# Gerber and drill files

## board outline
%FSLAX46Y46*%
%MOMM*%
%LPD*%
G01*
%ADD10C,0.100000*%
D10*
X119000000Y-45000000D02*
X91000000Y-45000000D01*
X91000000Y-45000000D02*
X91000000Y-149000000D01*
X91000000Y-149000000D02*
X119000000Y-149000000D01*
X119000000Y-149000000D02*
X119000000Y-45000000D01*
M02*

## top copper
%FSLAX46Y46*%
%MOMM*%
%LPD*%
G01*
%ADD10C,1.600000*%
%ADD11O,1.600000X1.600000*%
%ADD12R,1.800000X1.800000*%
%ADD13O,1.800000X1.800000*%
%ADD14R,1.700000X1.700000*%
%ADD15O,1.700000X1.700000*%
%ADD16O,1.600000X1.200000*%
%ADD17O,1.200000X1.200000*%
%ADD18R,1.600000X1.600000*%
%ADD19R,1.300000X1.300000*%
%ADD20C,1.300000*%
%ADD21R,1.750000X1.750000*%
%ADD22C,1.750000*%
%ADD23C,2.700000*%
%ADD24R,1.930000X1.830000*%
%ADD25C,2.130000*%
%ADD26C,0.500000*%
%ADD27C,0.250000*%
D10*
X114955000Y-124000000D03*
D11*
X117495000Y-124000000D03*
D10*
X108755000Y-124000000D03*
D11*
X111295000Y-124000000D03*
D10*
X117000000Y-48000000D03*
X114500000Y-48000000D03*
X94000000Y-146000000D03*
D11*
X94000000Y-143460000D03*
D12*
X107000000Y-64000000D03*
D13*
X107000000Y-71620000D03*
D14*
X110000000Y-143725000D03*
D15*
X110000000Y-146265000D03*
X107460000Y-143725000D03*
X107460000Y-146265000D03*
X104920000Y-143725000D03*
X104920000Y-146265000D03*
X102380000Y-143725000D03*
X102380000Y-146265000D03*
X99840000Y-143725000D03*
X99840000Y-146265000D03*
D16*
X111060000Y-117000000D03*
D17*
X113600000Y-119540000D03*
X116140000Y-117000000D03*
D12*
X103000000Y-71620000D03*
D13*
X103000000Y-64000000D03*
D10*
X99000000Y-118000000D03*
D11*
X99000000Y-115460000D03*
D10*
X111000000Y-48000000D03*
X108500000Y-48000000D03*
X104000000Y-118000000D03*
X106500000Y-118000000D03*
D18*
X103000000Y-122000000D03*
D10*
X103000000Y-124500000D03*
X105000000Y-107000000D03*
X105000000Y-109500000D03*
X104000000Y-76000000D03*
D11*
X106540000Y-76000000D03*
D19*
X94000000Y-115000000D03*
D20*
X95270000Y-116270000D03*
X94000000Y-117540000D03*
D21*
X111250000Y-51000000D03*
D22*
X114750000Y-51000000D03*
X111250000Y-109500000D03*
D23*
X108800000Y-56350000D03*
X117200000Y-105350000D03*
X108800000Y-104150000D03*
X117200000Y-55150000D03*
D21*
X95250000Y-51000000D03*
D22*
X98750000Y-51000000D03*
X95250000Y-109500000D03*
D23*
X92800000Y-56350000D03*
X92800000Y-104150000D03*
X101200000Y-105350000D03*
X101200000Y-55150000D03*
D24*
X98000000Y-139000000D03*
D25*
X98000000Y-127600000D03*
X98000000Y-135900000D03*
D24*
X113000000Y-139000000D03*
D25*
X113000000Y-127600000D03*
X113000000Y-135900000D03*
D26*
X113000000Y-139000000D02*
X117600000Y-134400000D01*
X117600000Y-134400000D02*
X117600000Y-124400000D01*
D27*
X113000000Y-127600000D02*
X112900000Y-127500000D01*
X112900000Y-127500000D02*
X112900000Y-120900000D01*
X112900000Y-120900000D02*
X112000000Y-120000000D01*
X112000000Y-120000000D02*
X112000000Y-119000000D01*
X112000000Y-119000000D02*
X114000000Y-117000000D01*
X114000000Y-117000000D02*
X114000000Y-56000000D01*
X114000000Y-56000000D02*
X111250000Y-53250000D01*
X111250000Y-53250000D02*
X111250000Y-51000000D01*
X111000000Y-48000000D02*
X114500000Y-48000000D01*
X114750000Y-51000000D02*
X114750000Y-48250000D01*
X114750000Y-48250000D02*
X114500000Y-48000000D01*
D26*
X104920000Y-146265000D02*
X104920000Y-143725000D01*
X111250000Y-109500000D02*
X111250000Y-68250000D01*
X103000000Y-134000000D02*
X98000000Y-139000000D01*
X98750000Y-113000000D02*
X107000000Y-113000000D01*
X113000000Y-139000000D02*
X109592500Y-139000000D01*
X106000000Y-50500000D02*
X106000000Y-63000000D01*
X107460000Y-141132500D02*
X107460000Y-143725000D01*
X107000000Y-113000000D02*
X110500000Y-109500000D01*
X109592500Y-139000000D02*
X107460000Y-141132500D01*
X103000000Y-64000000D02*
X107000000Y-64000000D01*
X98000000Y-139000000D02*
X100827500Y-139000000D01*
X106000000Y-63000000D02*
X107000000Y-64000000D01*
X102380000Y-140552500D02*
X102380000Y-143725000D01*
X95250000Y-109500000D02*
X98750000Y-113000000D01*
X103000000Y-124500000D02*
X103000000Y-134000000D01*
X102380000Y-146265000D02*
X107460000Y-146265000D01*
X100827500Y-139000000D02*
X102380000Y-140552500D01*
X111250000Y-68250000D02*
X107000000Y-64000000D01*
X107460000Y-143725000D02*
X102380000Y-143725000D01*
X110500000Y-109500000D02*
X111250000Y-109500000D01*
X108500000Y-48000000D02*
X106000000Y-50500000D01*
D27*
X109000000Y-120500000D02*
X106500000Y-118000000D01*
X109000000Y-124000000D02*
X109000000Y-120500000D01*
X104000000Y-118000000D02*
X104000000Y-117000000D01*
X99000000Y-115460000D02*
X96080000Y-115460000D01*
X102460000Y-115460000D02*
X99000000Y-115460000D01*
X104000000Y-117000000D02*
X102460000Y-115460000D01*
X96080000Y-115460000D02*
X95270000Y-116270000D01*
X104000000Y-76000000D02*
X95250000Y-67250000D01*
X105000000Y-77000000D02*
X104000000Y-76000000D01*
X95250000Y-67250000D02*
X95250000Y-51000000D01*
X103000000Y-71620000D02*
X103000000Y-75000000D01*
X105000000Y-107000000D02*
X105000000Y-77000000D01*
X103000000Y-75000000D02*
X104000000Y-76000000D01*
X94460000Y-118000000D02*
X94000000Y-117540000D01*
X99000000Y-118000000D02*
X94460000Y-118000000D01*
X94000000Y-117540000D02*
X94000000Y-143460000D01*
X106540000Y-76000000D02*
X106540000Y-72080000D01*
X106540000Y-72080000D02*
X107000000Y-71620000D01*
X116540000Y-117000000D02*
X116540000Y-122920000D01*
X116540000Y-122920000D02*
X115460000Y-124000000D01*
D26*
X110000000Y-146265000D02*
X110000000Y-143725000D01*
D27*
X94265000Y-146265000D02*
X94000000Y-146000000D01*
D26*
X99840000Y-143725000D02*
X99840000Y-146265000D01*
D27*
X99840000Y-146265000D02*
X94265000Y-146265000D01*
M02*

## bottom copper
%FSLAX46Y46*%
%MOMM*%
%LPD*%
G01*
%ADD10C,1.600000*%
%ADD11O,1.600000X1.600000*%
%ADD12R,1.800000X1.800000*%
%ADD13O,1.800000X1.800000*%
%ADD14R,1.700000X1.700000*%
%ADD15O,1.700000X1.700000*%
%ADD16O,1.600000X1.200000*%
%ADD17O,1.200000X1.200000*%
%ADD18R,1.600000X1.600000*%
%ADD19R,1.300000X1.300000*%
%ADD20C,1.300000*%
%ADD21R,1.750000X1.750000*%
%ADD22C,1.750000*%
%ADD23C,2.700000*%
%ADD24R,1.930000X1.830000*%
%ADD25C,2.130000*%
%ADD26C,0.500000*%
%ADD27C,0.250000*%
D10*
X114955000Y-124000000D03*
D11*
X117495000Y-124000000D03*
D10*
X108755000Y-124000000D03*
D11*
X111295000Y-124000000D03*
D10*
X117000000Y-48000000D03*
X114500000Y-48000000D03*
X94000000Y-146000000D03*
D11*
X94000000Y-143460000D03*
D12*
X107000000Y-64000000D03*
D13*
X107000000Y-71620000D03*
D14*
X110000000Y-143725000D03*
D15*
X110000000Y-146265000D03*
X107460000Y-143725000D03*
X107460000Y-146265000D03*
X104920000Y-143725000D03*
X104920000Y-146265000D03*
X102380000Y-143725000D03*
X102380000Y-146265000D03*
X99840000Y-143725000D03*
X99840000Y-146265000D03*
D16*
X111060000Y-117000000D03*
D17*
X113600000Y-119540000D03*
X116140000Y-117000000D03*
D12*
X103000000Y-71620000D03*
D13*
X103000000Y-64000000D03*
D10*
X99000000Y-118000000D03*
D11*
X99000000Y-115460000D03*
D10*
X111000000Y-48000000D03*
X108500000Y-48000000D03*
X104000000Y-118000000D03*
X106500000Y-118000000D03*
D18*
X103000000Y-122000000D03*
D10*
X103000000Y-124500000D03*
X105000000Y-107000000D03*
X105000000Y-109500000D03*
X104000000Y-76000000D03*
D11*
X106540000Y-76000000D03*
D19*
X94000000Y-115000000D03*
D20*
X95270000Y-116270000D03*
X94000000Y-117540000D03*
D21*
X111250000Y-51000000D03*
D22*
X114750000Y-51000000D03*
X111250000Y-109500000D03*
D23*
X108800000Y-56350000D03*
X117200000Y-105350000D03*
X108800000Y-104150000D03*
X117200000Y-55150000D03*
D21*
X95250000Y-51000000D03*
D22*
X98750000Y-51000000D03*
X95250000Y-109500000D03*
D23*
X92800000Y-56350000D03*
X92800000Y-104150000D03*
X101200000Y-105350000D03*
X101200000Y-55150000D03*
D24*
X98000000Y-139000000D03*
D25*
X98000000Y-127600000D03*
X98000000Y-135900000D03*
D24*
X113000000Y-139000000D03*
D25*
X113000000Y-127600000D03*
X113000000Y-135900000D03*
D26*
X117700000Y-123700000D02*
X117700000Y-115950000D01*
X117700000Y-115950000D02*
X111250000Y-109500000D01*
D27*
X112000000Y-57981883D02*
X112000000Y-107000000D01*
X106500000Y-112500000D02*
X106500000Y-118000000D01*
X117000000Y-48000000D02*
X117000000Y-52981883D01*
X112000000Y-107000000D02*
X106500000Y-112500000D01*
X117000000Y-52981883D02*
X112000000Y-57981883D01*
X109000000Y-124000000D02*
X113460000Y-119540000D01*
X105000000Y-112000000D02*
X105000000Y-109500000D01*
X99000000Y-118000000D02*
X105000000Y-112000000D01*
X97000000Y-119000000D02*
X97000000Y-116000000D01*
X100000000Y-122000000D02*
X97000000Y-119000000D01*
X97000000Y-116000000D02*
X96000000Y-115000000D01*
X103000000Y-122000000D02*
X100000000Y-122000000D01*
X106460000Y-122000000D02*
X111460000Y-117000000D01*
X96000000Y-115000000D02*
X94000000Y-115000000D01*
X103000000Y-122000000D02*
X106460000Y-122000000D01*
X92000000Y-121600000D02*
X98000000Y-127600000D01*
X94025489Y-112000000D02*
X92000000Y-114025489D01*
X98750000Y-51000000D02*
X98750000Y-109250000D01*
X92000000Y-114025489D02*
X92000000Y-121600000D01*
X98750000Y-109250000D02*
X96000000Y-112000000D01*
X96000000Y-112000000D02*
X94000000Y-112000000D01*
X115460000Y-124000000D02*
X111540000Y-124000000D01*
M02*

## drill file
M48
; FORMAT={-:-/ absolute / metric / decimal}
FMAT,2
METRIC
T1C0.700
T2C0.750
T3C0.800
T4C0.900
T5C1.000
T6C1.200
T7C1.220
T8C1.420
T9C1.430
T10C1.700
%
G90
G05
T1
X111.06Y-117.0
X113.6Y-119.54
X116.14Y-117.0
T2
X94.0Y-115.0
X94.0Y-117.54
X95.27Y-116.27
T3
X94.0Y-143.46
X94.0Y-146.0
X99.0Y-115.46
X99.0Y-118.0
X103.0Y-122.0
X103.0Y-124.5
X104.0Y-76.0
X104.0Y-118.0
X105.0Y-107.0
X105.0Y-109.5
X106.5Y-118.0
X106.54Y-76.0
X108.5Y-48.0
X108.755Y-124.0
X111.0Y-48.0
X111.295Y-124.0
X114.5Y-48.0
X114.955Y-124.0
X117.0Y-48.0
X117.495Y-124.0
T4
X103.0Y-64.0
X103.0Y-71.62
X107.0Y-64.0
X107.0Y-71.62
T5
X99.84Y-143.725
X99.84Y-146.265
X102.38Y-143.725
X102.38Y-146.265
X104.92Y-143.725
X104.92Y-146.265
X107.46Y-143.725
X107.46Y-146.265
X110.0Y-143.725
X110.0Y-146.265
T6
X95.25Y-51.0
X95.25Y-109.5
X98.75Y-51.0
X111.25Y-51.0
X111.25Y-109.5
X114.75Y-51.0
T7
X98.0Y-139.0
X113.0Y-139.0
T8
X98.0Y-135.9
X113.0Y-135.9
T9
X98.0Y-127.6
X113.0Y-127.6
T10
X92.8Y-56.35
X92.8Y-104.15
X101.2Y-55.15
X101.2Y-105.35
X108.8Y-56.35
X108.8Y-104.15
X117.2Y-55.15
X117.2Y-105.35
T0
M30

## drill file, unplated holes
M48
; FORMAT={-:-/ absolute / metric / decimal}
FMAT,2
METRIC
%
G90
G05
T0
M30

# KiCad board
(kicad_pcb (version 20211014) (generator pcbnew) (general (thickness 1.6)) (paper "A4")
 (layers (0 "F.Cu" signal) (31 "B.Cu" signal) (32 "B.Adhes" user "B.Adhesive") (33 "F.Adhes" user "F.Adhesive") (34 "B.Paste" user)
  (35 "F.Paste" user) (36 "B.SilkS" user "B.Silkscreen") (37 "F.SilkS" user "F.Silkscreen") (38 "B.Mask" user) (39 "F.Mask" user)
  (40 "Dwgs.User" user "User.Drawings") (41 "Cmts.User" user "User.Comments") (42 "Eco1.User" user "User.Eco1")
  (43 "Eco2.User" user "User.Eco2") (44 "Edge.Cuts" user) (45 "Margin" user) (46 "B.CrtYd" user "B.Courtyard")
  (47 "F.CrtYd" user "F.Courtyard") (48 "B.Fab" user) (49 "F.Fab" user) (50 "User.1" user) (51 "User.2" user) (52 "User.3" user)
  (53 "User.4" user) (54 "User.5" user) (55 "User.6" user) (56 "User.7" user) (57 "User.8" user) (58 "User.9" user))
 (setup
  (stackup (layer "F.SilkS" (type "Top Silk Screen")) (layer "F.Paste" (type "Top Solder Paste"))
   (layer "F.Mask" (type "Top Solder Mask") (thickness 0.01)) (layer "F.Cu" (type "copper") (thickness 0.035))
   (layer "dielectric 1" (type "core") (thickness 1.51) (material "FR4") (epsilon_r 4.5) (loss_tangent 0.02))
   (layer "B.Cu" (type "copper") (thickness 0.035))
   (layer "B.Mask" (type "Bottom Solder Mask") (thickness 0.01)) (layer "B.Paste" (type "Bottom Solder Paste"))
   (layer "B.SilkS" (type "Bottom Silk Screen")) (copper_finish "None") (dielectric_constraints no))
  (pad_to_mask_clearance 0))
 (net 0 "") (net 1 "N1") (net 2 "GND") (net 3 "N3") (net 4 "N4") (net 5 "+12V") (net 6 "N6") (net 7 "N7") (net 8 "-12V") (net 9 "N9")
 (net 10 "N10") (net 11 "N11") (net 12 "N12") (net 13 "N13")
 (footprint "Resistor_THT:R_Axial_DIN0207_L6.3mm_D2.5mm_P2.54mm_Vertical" (layer "F.Cu") (at 114.955 124)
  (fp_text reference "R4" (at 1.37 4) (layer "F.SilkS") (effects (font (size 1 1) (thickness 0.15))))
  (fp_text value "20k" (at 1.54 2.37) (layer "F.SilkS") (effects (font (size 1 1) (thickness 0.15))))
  (pad "1" thru_hole circle (at 0 0) (size 1.6 1.6) (drill 0.8) (layers *.Cu *.Mask) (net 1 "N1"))
  (pad "2" thru_hole oval (at 2.54 0) (size 1.6 1.6) (drill 0.8) (layers *.Cu *.Mask) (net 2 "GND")))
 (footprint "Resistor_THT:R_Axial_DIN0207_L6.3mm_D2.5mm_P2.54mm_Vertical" (layer "F.Cu") (at 108.755 124)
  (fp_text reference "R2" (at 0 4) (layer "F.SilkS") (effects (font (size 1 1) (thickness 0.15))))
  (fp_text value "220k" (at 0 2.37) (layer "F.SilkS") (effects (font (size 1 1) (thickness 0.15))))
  (pad "1" thru_hole circle (at 0 0) (size 1.6 1.6) (drill 0.8) (layers *.Cu *.Mask) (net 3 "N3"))
  (pad "2" thru_hole oval (at 2.54 0) (size 1.6 1.6) (drill 0.8) (layers *.Cu *.Mask) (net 1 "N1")))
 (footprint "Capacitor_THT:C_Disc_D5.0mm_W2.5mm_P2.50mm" (layer "F.Cu") (at 117 48 180)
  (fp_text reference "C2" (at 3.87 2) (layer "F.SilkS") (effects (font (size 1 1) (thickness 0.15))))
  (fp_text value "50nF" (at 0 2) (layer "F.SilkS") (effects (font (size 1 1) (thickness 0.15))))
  (pad "1" thru_hole circle (at 0 0 180) (size 1.6 1.6) (drill 0.8) (layers *.Cu *.Mask) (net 3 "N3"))
  (pad "2" thru_hole circle (at 2.5 0 180) (size 1.6 1.6) (drill 0.8) (layers *.Cu *.Mask) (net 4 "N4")))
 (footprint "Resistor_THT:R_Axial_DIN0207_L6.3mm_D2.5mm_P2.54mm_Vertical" (layer "F.Cu") (at 94 146 90)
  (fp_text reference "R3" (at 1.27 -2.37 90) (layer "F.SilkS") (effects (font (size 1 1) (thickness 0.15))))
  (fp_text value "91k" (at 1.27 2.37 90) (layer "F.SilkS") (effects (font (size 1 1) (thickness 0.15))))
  (pad "1" thru_hole circle (at 0 0 90) (size 1.6 1.6) (drill 0.8) (layers *.Cu *.Mask) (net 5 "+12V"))
  (pad "2" thru_hole oval (at 2.54 0 90) (size 1.6 1.6) (drill 0.8) (layers *.Cu *.Mask) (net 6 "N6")))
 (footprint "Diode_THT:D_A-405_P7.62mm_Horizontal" (layer "F.Cu") (at 107 64 -90)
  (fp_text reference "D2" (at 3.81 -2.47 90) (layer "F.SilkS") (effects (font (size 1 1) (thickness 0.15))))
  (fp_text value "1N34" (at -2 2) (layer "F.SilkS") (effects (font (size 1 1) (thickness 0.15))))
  (pad "1" thru_hole rect (at 0 0 270) (size 1.8 1.8) (drill 0.9) (layers *.Cu *.Mask) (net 2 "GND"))
  (pad "2" thru_hole oval (at 7.62 0 270) (size 1.8 1.8) (drill 0.9) (layers *.Cu *.Mask) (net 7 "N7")))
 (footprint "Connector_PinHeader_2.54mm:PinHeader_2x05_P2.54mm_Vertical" (layer "F.Cu") (at 110 143.725 -90)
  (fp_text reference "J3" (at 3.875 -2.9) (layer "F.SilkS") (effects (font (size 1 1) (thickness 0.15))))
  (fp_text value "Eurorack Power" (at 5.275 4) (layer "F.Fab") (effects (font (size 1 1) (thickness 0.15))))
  (pad "1" thru_hole rect (at 0 0 270) (size 1.7 1.7) (drill 1) (layers *.Cu *.Mask) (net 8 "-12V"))
  (pad "2" thru_hole oval (at 2.54 0 270) (size 1.7 1.7) (drill 1) (layers *.Cu *.Mask) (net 8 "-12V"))
  (pad "3" thru_hole oval (at 0 2.54 270) (size 1.7 1.7) (drill 1) (layers *.Cu *.Mask) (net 2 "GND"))
  (pad "4" thru_hole oval (at 2.54 2.54 270) (size 1.7 1.7) (drill 1) (layers *.Cu *.Mask) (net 2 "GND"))
  (pad "5" thru_hole oval (at 0 5.08 270) (size 1.7 1.7) (drill 1) (layers *.Cu *.Mask) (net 2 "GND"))
  (pad "6" thru_hole oval (at 2.54 5.08 270) (size 1.7 1.7) (drill 1) (layers *.Cu *.Mask) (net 2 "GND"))
  (pad "7" thru_hole oval (at 0 7.62 270) (size 1.7 1.7) (drill 1) (layers *.Cu *.Mask) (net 2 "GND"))
  (pad "8" thru_hole oval (at 2.54 7.62 270) (size 1.7 1.7) (drill 1) (layers *.Cu *.Mask) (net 2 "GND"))
  (pad "9" thru_hole oval (at 0 10.16 270) (size 1.7 1.7) (drill 1) (layers *.Cu *.Mask) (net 5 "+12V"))
  (pad "10" thru_hole oval (at 2.54 10.16 270) (size 1.7 1.7) (drill 1) (layers *.Cu *.Mask) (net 5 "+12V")))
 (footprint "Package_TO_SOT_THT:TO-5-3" (layer "F.Cu") (at 111.06 117)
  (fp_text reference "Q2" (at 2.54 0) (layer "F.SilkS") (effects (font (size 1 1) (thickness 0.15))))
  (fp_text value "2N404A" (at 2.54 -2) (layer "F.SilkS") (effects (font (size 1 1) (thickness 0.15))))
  (pad "1" thru_hole oval (at 0 0) (size 1.6 1.2) (drill 0.7) (layers *.Cu *.Mask) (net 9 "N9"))
  (pad "2" thru_hole oval (at 2.54 2.54) (size 1.2 1.2) (drill 0.7) (layers *.Cu *.Mask) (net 3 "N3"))
  (pad "3" thru_hole oval (at 5.08 0) (size 1.2 1.2) (drill 0.7) (layers *.Cu *.Mask) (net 1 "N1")))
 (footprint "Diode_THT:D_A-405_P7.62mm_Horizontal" (layer "F.Cu") (at 103 71.62 90)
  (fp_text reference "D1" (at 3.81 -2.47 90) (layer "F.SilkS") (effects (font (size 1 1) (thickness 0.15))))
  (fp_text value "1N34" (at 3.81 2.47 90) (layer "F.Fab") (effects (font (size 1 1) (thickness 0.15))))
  (pad "1" thru_hole rect (at 0 0 90) (size 1.8 1.8) (drill 0.9) (layers *.Cu *.Mask) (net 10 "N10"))
  (pad "2" thru_hole oval (at 7.62 0 90) (size 1.8 1.8) (drill 0.9) (layers *.Cu *.Mask) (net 2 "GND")))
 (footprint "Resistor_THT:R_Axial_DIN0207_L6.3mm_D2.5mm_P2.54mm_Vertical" (layer "F.Cu") (at 99 118 90)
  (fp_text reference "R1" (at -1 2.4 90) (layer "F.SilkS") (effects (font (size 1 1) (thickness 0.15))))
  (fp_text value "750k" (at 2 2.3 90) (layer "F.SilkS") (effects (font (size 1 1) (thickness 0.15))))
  (pad "1" thru_hole circle (at 0 0 90) (size 1.6 1.6) (drill 0.8) (layers *.Cu *.Mask) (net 6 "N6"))
  (pad "2" thru_hole oval (at 2.54 0 90) (size 1.6 1.6) (drill 0.8) (layers *.Cu *.Mask) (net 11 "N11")))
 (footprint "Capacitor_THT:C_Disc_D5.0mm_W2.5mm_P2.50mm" (layer "F.Cu") (at 111 48 180)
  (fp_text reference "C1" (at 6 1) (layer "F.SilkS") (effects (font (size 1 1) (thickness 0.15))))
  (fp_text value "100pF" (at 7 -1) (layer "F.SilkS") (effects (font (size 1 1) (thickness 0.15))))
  (pad "1" thru_hole circle (at 0 0 180) (size 1.6 1.6) (drill 0.8) (layers *.Cu *.Mask) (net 4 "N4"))
  (pad "2" thru_hole circle (at 2.5 0 180) (size 1.6 1.6) (drill 0.8) (layers *.Cu *.Mask) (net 2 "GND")))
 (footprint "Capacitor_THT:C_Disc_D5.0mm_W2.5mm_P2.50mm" (layer "F.Cu") (at 104 118)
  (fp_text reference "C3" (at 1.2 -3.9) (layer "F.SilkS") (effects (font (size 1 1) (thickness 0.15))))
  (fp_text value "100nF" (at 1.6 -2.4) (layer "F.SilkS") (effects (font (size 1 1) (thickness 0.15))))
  (pad "1" thru_hole circle (at 0 0) (size 1.6 1.6) (drill 0.8) (layers *.Cu *.Mask) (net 11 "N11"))
  (pad "2" thru_hole circle (at 2.5 0) (size 1.6 1.6) (drill 0.8) (layers *.Cu *.Mask) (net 3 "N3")))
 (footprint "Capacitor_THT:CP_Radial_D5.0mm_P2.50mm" (layer "F.Cu") (at 103 122 -90)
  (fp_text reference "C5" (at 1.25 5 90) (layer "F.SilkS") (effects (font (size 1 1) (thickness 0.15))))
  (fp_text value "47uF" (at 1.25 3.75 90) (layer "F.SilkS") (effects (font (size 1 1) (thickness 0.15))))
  (pad "1" thru_hole rect (at 0 0 270) (size 1.6 1.6) (drill 0.8) (layers *.Cu *.Mask) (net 9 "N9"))
  (pad "2" thru_hole circle (at 2.5 0 270) (size 1.6 1.6) (drill 0.8) (layers *.Cu *.Mask) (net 2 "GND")))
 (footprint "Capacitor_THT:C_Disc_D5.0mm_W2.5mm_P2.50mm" (layer "F.Cu") (at 105 107 -90)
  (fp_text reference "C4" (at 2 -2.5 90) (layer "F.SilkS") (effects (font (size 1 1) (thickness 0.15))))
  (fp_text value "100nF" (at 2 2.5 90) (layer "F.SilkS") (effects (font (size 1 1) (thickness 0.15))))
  (pad "1" thru_hole circle (at 0 0 270) (size 1.6 1.6) (drill 0.8) (layers *.Cu *.Mask) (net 10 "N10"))
  (pad "2" thru_hole circle (at 2.5 0 270) (size 1.6 1.6) (drill 0.8) (layers *.Cu *.Mask) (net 6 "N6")))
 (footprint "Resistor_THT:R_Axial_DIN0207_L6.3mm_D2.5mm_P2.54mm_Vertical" (layer "F.Cu") (at 104 76)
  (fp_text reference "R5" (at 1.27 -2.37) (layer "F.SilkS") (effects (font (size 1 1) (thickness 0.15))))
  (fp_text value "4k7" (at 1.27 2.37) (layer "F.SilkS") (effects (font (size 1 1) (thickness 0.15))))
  (pad "1" thru_hole circle (at 0 0) (size 1.6 1.6) (drill 0.8) (layers *.Cu *.Mask) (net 10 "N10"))
  (pad "2" thru_hole oval (at 2.54 0) (size 1.6 1.6) (drill 0.8) (layers *.Cu *.Mask) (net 7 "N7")))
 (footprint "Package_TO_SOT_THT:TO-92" (layer "F.Cu") (at 94 115 -90)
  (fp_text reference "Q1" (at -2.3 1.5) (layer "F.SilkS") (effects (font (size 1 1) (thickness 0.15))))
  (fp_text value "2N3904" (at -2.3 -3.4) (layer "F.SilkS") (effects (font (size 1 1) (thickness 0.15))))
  (pad "1" thru_hole rect (at 0 0 270) (size 1.3 1.3) (drill 0.75) (layers *.Cu *.Mask) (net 9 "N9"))
  (pad "2" thru_hole circle (at 1.27 -1.27 270) (size 1.3 1.3) (drill 0.75) (layers *.Cu *.Mask) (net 11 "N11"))
  (pad "3" thru_hole circle (at 2.54 0 270) (size 1.3 1.3) (drill 0.75) (layers *.Cu *.Mask) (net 6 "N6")))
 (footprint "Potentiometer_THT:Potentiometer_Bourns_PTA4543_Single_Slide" (layer "B.Cu") (at 111.25 51 -90)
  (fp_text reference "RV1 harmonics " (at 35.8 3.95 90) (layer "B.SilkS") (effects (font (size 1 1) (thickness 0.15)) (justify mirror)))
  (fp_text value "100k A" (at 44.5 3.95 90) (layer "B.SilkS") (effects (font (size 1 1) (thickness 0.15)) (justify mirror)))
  (pad "1" thru_hole rect (at 0 0 270) (size 1.75 1.75) (drill 1.2) (layers *.Cu *.Mask) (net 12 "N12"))
  (pad "2" thru_hole circle (at 0 -3.5 270) (size 1.75 1.75) (drill 1.2) (layers *.Cu *.Mask) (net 4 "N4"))
  (pad "3" thru_hole circle (at 58.5 0 270) (size 1.75 1.75) (drill 1.2) (layers *.Cu *.Mask) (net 2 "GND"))
  (pad "MP" thru_hole circle (at 5.35 2.45 270) (size 2.7 2.7) (drill 1.7) (layers *.Cu *.Mask))
  (pad "MP" thru_hole circle (at 54.35 -5.95 270) (size 2.7 2.7) (drill 1.7) (layers *.Cu *.Mask))
  (pad "MP" thru_hole circle (at 53.15 2.45 270) (size 2.7 2.7) (drill 1.7) (layers *.Cu *.Mask))
  (pad "MP" thru_hole circle (at 4.15 -5.95 270) (size 2.7 2.7) (drill 1.7) (layers *.Cu *.Mask)))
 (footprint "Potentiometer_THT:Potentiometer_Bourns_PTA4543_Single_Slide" (layer "B.Cu") (at 95.25 51 -90)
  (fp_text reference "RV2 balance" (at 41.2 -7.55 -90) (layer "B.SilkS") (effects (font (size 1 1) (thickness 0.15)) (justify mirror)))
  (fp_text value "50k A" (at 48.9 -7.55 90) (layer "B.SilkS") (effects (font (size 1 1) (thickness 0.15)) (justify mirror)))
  (pad "1" thru_hole rect (at 0 0 270) (size 1.75 1.75) (drill 1.2) (layers *.Cu *.Mask) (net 10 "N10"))
  (pad "2" thru_hole circle (at 0 -3.5 270) (size 1.75 1.75) (drill 1.2) (layers *.Cu *.Mask) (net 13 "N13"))
  (pad "3" thru_hole circle (at 58.5 0 270) (size 1.75 1.75) (drill 1.2) (layers *.Cu *.Mask) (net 2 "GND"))
  (pad "MP" thru_hole circle (at 5.35 2.45 270) (size 2.7 2.7) (drill 1.7) (layers *.Cu *.Mask))
  (pad "MP" thru_hole circle (at 53.15 2.45 270) (size 2.7 2.7) (drill 1.7) (layers *.Cu *.Mask))
  (pad "MP" thru_hole circle (at 54.35 -5.95 270) (size 2.7 2.7) (drill 1.7) (layers *.Cu *.Mask))
  (pad "MP" thru_hole circle (at 4.15 -5.95 270) (size 2.7 2.7) (drill 1.7) (layers *.Cu *.Mask)))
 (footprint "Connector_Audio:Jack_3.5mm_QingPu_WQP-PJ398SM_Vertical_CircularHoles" (layer "B.Cu") (at 98 139)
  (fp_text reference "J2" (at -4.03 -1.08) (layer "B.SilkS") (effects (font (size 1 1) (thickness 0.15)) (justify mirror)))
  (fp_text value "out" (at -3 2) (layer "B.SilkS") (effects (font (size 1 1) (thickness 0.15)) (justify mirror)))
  (pad "S" thru_hole rect (at 0 0 180) (size 1.93 1.83) (drill 1.22) (layers *.Cu *.Mask) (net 2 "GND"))
  (pad "T" thru_hole circle (at 0 -11.4 180) (size 2.13 2.13) (drill 1.43) (layers *.Cu *.Mask) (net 13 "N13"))
  (pad "TN" thru_hole circle (at 0 -3.1 180) (size 2.13 2.13) (drill 1.42) (layers *.Cu *.Mask))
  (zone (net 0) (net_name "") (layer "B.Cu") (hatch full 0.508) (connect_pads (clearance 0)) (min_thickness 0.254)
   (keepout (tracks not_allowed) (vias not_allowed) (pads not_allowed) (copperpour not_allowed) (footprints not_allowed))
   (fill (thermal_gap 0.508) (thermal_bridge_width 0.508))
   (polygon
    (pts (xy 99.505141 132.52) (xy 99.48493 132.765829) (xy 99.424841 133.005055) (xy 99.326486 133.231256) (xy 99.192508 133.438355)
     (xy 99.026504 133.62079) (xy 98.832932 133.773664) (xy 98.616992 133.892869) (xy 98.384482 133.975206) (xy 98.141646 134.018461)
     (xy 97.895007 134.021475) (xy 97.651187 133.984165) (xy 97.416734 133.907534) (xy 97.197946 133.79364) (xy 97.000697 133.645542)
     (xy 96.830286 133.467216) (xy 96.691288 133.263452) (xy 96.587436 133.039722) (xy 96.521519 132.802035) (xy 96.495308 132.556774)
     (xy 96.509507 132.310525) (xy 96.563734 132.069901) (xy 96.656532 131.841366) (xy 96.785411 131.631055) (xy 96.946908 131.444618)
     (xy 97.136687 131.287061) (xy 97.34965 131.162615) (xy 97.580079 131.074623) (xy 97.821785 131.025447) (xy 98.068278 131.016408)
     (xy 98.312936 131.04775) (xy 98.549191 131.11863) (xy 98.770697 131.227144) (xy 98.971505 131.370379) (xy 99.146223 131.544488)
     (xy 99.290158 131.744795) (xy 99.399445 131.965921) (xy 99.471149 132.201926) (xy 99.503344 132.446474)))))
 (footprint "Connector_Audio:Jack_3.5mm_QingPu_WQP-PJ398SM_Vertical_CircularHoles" (layer "B.Cu") (at 113 139)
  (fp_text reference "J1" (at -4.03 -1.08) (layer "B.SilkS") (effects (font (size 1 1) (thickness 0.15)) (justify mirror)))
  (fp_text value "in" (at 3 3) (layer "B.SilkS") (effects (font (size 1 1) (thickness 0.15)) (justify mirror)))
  (pad "S" thru_hole rect (at 0 0 180) (size 1.93 1.83) (drill 1.22) (layers *.Cu *.Mask) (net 2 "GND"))
  (pad "T" thru_hole circle (at 0 -11.4 180) (size 2.13 2.13) (drill 1.43) (layers *.Cu *.Mask) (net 12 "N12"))
  (pad "TN" thru_hole circle (at 0 -3.1 180) (size 2.13 2.13) (drill 1.42) (layers *.Cu *.Mask))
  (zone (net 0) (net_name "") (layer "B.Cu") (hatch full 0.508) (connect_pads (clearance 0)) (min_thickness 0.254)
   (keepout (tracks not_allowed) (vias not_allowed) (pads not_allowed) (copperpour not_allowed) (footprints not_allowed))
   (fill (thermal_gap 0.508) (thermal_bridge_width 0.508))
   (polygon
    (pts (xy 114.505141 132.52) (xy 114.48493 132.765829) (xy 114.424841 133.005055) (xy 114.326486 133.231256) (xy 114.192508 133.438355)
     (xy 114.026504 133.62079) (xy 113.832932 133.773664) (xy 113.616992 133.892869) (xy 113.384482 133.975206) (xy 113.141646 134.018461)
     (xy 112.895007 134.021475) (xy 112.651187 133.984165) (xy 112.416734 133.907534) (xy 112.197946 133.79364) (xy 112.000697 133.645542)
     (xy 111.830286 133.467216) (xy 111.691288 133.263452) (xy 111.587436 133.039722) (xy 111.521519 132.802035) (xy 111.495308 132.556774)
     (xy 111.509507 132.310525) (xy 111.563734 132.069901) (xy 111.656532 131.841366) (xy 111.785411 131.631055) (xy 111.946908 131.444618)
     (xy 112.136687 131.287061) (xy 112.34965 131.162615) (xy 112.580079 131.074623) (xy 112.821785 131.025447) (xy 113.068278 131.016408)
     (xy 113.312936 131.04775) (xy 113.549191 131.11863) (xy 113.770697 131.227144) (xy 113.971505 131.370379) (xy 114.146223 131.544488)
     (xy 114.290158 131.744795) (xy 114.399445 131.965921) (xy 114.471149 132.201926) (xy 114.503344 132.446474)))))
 (gr_rect (start 119 45) (end 91 149) (layer "Edge.Cuts") (width 0.1) (fill none))
 (segment (start 111 48) (end 114.5 48) (width 0.25) (layer "F.Cu") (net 4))
 (segment (start 114.75 51) (end 114.75 48.25) (width 0.25) (layer "F.Cu") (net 4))
 (segment (start 114.75 48.25) (end 114.5 48) (width 0.25) (layer "F.Cu") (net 4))
 (segment (start 104.92 146.265) (end 104.92 143.725) (width 0.5) (layer "F.Cu") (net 2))
 (segment (start 111.25 109.5) (end 111.25 68.25) (width 0.5) (layer "F.Cu") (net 2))
 (segment (start 103 134) (end 98 139) (width 0.5) (layer "F.Cu") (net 2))
 (segment (start 98.75 113) (end 107 113) (width 0.5) (layer "F.Cu") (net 2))
 (segment (start 113 139) (end 109.5925 139) (width 0.5) (layer "F.Cu") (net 2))
 (segment (start 106 50.5) (end 106 63) (width 0.5) (layer "F.Cu") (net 2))
 (segment (start 117.6 134.4) (end 117.6 124.4) (width 0.5) (layer "F.Cu") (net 2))
 (segment (start 107.46 141.1325) (end 107.46 143.725) (width 0.5) (layer "F.Cu") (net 2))
 (segment (start 107 113) (end 110.5 109.5) (width 0.5) (layer "F.Cu") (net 2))
 (segment (start 109.5925 139) (end 107.46 141.1325) (width 0.5) (layer "F.Cu") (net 2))
 (segment (start 103 64) (end 107 64) (width 0.5) (layer "F.Cu") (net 2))
 (segment (start 98 139) (end 100.8275 139) (width 0.5) (layer "F.Cu") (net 2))
 (segment (start 106 63) (end 107 64) (width 0.5) (layer "F.Cu") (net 2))
 (segment (start 102.38 140.5525) (end 102.38 143.725) (width 0.5) (layer "F.Cu") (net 2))
 (segment (start 95.25 109.5) (end 98.75 113) (width 0.5) (layer "F.Cu") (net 2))
 (segment (start 103 124.5) (end 103 134) (width 0.5) (layer "F.Cu") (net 2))
 (segment (start 102.38 146.265) (end 107.46 146.265) (width 0.5) (layer "F.Cu") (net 2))
 (segment (start 100.8275 139) (end 102.38 140.5525) (width 0.5) (layer "F.Cu") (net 2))
 (segment (start 111.25 68.25) (end 107 64) (width 0.5) (layer "F.Cu") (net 2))
 (segment (start 107.46 143.725) (end 102.38 143.725) (width 0.5) (layer "F.Cu") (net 2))
 (segment (start 113 139) (end 117.6 134.4) (width 0.5) (layer "F.Cu") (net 2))
 (segment (start 110.5 109.5) (end 111.25 109.5) (width 0.5) (layer "F.Cu") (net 2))
 (segment (start 108.5 48) (end 106 50.5) (width 0.5) (layer "F.Cu") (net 2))
 (segment (start 117.7 115.95) (end 111.25 109.5) (width 0.5) (layer "B.Cu") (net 2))
 (segment (start 117.7 123.7) (end 117.7 115.95) (width 0.5) (layer "B.Cu") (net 2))
 (segment (start 109 120.5) (end 106.5 118) (width 0.25) (layer "F.Cu") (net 3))
 (segment (start 109 124) (end 109 120.5) (width 0.25) (layer "F.Cu") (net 3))
 (segment (start 112 57.981883) (end 112 107) (width 0.25) (layer "B.Cu") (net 3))
 (segment (start 106.5 112.5) (end 106.5 118) (width 0.25) (layer "B.Cu") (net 3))
 (segment (start 117 48) (end 117 52.981883) (width 0.25) (layer "B.Cu") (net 3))
 (segment (start 112 107) (end 106.5 112.5) (width 0.25) (layer "B.Cu") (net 3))
 (segment (start 117 52.981883) (end 112 57.981883) (width 0.25) (layer "B.Cu") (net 3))
 (segment (start 109 124) (end 113.46 119.54) (width 0.25) (layer "B.Cu") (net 3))
 (segment (start 104 118) (end 104 117) (width 0.25) (layer "F.Cu") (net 11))
 (segment (start 99 115.46) (end 96.08 115.46) (width 0.25) (layer "F.Cu") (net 11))
 (segment (start 102.46 115.46) (end 99 115.46) (width 0.25) (layer "F.Cu") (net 11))
 (segment (start 104 117) (end 102.46 115.46) (width 0.25) (layer "F.Cu") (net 11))
 (segment (start 96.08 115.46) (end 95.27 116.27) (width 0.25) (layer "F.Cu") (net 11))
 (segment (start 104 76) (end 95.25 67.25) (width 0.25) (layer "F.Cu") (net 10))
 (segment (start 105 77) (end 104 76) (width 0.25) (layer "F.Cu") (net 10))
 (segment (start 95.25 67.25) (end 95.25 51) (width 0.25) (layer "F.Cu") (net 10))
 (segment (start 103 71.62) (end 103 75) (width 0.25) (layer "F.Cu") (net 10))
 (segment (start 105 107) (end 105 77) (width 0.25) (layer "F.Cu") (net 10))
 (segment (start 103 75) (end 104 76) (width 0.25) (layer "F.Cu") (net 10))
 (segment (start 94.46 118) (end 94 117.54) (width 0.25) (layer "F.Cu") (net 6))
 (segment (start 99 118) (end 94.46 118) (width 0.25) (layer "F.Cu") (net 6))
 (segment (start 94 117.54) (end 94 143.46) (width 0.25) (layer "F.Cu") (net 6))
 (segment (start 105 112) (end 105 109.5) (width 0.25) (layer "B.Cu") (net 6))
 (segment (start 99 118) (end 105 112) (width 0.25) (layer "B.Cu") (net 6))
 (segment (start 97 119) (end 97 116) (width 0.25) (layer "B.Cu") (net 9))
 (segment (start 100 122) (end 97 119) (width 0.25) (layer "B.Cu") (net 9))
 (segment (start 97 116) (end 96 115) (width 0.25) (layer "B.Cu") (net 9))
 (segment (start 103 122) (end 100 122) (width 0.25) (layer "B.Cu") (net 9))
 (segment (start 106.46 122) (end 111.46 117) (width 0.25) (layer "B.Cu") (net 9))
 (segment (start 96 115) (end 94 115) (width 0.25) (layer "B.Cu") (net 9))
 (segment (start 103 122) (end 106.46 122) (width 0.25) (layer "B.Cu") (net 9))
 (segment (start 106.54 76) (end 106.54 72.08) (width 0.25) (layer "F.Cu") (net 7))
 (segment (start 106.54 72.08) (end 107 71.62) (width 0.25) (layer "F.Cu") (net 7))
 (segment (start 112.9 127.5) (end 112.9 120.9) (width 0.25) (layer "F.Cu") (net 12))
 (segment (start 111.25 53.25) (end 111.25 51) (width 0.25) (layer "F.Cu") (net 12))
 (segment (start 112 119) (end 114 117) (width 0.25) (layer "F.Cu") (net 12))
 (segment (start 112 120) (end 112 119) (width 0.25) (layer "F.Cu") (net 12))
 (segment (start 114 117) (end 114 56) (width 0.25) (layer "F.Cu") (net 12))
 (segment (start 113 127.6) (end 112.9 127.5) (width 0.25) (layer "F.Cu") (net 12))
 (segment (start 114 56) (end 111.25 53.25) (width 0.25) (layer "F.Cu") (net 12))
 (segment (start 112.9 120.9) (end 112 120) (width 0.25) (layer "F.Cu") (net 12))
 (segment (start 92 121.6) (end 98 127.6) (width 0.25) (layer "B.Cu") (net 13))
 (segment (start 94.025489 112) (end 92 114.025489) (width 0.25) (layer "B.Cu") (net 13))
 (segment (start 98.75 51) (end 98.75 109.25) (width 0.25) (layer "B.Cu") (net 13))
 (segment (start 92 114.025489) (end 92 121.6) (width 0.25) (layer "B.Cu") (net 13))
 (segment (start 98.75 109.25) (end 96 112) (width 0.25) (layer "B.Cu") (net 13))
 (segment (start 96 112) (end 94 112) (width 0.25) (layer "B.Cu") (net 13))
 (segment (start 116.54 117) (end 116.54 122.92) (width 0.25) (layer "F.Cu") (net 1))
 (segment (start 116.54 122.92) (end 115.46 124) (width 0.25) (layer "F.Cu") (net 1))
 (segment (start 115.46 124) (end 111.54 124) (width 0.25) (layer "B.Cu") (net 1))
 (segment (start 110 146.265) (end 110 143.725) (width 0.5) (layer "F.Cu") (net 8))
 (segment (start 94.265 146.265) (end 94 146) (width 0.25) (layer "F.Cu") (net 5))
 (segment (start 99.84 143.725) (end 99.84 146.265) (width 0.5) (layer "F.Cu") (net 5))
 (segment (start 99.84 146.265) (end 94.265 146.265) (width 0.25) (layer "F.Cu") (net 5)))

